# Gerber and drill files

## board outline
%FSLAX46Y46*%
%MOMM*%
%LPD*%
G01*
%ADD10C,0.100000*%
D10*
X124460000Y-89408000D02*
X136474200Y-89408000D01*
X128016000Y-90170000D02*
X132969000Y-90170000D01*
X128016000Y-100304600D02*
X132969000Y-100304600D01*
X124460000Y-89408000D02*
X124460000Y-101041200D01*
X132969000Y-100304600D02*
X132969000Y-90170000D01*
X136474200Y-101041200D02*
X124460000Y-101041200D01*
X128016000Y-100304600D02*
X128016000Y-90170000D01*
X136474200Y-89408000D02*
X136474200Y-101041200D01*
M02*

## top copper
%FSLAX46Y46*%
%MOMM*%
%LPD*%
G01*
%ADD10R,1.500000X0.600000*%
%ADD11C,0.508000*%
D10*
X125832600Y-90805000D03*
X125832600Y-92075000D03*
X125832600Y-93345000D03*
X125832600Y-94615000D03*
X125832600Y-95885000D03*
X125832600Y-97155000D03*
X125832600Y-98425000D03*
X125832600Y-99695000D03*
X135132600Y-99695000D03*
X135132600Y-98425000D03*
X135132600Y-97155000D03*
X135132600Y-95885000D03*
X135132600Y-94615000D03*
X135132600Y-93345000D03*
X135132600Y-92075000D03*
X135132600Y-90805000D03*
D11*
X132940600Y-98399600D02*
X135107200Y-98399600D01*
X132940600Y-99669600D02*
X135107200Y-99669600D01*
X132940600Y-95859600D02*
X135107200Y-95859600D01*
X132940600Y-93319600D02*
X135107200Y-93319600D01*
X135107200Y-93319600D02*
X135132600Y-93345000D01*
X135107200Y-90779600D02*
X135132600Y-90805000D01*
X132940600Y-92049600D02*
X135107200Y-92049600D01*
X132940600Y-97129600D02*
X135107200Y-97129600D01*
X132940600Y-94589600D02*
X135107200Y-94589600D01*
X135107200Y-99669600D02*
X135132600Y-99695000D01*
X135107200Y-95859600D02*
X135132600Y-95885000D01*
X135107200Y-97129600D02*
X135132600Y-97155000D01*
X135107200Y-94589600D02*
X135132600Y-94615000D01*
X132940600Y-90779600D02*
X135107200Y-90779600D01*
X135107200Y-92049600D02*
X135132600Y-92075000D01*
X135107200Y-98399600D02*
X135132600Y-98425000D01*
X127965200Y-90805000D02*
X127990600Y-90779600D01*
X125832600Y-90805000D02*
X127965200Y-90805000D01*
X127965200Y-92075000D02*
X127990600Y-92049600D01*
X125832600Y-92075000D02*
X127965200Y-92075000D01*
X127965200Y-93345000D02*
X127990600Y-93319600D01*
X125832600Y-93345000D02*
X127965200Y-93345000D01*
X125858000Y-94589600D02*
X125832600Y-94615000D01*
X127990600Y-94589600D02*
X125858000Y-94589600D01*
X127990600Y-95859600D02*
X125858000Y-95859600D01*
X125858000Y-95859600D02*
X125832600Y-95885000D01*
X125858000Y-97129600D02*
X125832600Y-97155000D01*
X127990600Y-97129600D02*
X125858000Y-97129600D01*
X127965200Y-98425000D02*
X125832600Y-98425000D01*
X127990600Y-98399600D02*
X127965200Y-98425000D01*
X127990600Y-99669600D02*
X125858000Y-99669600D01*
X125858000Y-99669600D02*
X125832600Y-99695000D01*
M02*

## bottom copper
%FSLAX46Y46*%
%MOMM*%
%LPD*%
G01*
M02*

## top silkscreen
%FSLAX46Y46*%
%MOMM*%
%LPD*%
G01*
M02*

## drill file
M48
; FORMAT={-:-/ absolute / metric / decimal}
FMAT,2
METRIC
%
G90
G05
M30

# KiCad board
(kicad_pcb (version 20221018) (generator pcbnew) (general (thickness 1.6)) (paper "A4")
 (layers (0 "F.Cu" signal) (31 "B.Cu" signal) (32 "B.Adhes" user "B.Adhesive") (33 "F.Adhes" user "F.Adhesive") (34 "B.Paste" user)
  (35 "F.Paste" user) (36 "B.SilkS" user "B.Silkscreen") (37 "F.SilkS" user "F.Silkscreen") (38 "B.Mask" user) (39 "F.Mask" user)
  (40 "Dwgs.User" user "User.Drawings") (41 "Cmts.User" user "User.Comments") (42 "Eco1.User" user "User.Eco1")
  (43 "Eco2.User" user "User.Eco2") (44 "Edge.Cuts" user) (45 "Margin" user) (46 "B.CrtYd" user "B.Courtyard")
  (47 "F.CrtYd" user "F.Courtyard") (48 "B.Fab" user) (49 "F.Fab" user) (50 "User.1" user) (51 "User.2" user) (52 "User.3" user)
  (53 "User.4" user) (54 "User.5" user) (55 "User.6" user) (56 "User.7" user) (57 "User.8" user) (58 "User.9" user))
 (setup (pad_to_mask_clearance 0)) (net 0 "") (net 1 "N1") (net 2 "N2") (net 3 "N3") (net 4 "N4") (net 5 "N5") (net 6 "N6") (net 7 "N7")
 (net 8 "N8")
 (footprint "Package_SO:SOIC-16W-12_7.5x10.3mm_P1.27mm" (layer "F.Cu") (at 130.4826 95.25)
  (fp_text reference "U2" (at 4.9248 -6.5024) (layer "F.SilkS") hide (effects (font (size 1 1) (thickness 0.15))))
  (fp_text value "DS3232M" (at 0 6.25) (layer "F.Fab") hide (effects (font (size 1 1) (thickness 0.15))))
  (pad "1" smd rect (at -4.65 -4.445) (size 1.5 0.6) (layers "F.Cu" "F.Paste" "F.Mask") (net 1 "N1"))
  (pad "2" smd rect (at -4.65 -3.175) (size 1.5 0.6) (layers "F.Cu" "F.Paste" "F.Mask") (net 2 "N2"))
  (pad "3" smd rect (at -4.65 -1.905) (size 1.5 0.6) (layers "F.Cu" "F.Paste" "F.Mask") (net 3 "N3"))
  (pad "4" smd rect (at -4.65 -0.635) (size 1.5 0.6) (layers "F.Cu" "F.Paste" "F.Mask"))
  (pad "5" smd rect (at -4.65 0.635) (size 1.5 0.6) (layers "F.Cu" "F.Paste" "F.Mask"))
  (pad "6" smd rect (at -4.65 1.905) (size 1.5 0.6) (layers "F.Cu" "F.Paste" "F.Mask") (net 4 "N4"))
  (pad "7" smd rect (at -4.65 3.175) (size 1.5 0.6) (layers "F.Cu" "F.Paste" "F.Mask") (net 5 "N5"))
  (pad "8" smd rect (at -4.65 4.445) (size 1.5 0.6) (layers "F.Cu" "F.Paste" "F.Mask") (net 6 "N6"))
  (pad "9" smd rect (at 4.65 4.445) (size 1.5 0.6) (layers "F.Cu" "F.Paste" "F.Mask"))
  (pad "10" smd rect (at 4.65 3.175) (size 1.5 0.6) (layers "F.Cu" "F.Paste" "F.Mask"))
  (pad "11" smd rect (at 4.65 1.905) (size 1.5 0.6) (layers "F.Cu" "F.Paste" "F.Mask"))
  (pad "12" smd rect (at 4.65 0.635) (size 1.5 0.6) (layers "F.Cu" "F.Paste" "F.Mask"))
  (pad "13" smd rect (at 4.65 -0.635) (size 1.5 0.6) (layers "F.Cu" "F.Paste" "F.Mask"))
  (pad "14" smd rect (at 4.65 -1.905) (size 1.5 0.6) (layers "F.Cu" "F.Paste" "F.Mask"))
  (pad "15" smd rect (at 4.65 -3.175) (size 1.5 0.6) (layers "F.Cu" "F.Paste" "F.Mask"))
  (pad "16" smd rect (at 4.65 -4.445) (size 1.5 0.6) (layers "F.Cu" "F.Paste" "F.Mask")))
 (gr_line (start 124.46 89.408) (end 136.4742 89.408) (stroke (width 0.1) (type default)) (layer "Edge.Cuts"))
 (gr_line (start 128.016 90.17) (end 132.969 90.17) (stroke (width 0.1) (type default)) (layer "Edge.Cuts"))
 (gr_line (start 128.016 100.3046) (end 132.969 100.3046) (stroke (width 0.1) (type default)) (layer "Edge.Cuts"))
 (gr_line (start 124.46 89.408) (end 124.46 101.0412) (stroke (width 0.1) (type default)) (layer "Edge.Cuts"))
 (gr_line (start 132.969 100.3046) (end 132.969 90.17) (stroke (width 0.1) (type default)) (layer "Edge.Cuts"))
 (gr_line (start 136.4742 101.0412) (end 124.46 101.0412) (stroke (width 0.1) (type default)) (layer "Edge.Cuts"))
 (gr_line (start 128.016 100.3046) (end 128.016 90.17) (stroke (width 0.1) (type default)) (layer "Edge.Cuts"))
 (gr_line (start 136.4742 89.408) (end 136.4742 101.0412) (stroke (width 0.1) (type default)) (layer "Edge.Cuts"))
 (segment (start 132.9406 98.3996) (end 135.1072 98.3996) (width 0.508) (layer "F.Cu") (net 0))
 (segment (start 132.9406 99.6696) (end 135.1072 99.6696) (width 0.508) (layer "F.Cu") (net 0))
 (segment (start 132.9406 95.8596) (end 135.1072 95.8596) (width 0.508) (layer "F.Cu") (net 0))
 (segment (start 132.9406 93.3196) (end 135.1072 93.3196) (width 0.508) (layer "F.Cu") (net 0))
 (segment (start 135.1072 93.3196) (end 135.1326 93.345) (width 0.508) (layer "F.Cu") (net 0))
 (segment (start 135.1072 90.7796) (end 135.1326 90.805) (width 0.508) (layer "F.Cu") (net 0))
 (segment (start 132.9406 92.0496) (end 135.1072 92.0496) (width 0.508) (layer "F.Cu") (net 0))
 (segment (start 132.9406 97.1296) (end 135.1072 97.1296) (width 0.508) (layer "F.Cu") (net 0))
 (segment (start 132.9406 94.5896) (end 135.1072 94.5896) (width 0.508) (layer "F.Cu") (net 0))
 (segment (start 135.1072 99.6696) (end 135.1326 99.695) (width 0.508) (layer "F.Cu") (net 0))
 (segment (start 135.1072 95.8596) (end 135.1326 95.885) (width 0.508) (layer "F.Cu") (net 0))
 (segment (start 135.1072 97.1296) (end 135.1326 97.155) (width 0.508) (layer "F.Cu") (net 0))
 (segment (start 135.1072 94.5896) (end 135.1326 94.615) (width 0.508) (layer "F.Cu") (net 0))
 (segment (start 132.9406 90.7796) (end 135.1072 90.7796) (width 0.508) (layer "F.Cu") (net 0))
 (segment (start 135.1072 92.0496) (end 135.1326 92.075) (width 0.508) (layer "F.Cu") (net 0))
 (segment (start 135.1072 98.3996) (end 135.1326 98.425) (width 0.508) (layer "F.Cu") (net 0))
 (segment (start 127.9652 90.805) (end 127.9906 90.7796) (width 0.508) (layer "F.Cu") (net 1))
 (segment (start 125.8326 90.805) (end 127.9652 90.805) (width 0.508) (layer "F.Cu") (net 1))
 (segment (start 127.9652 92.075) (end 127.9906 92.0496) (width 0.508) (layer "F.Cu") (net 2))
 (segment (start 125.8326 92.075) (end 127.9652 92.075) (width 0.508) (layer "F.Cu") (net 2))
 (segment (start 127.9652 93.345) (end 127.9906 93.3196) (width 0.508) (layer "F.Cu") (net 3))
 (segment (start 125.8326 93.345) (end 127.9652 93.345) (width 0.508) (layer "F.Cu") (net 3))
 (segment (start 125.858 94.5896) (end 125.8326 94.615) (width 0.508) (layer "F.Cu") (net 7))
 (segment (start 127.9906 94.5896) (end 125.858 94.5896) (width 0.508) (layer "F.Cu") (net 7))
 (segment (start 127.9906 95.8596) (end 125.858 95.8596) (width 0.508) (layer "F.Cu") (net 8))
 (segment (start 125.858 95.8596) (end 125.8326 95.885) (width 0.508) (layer "F.Cu") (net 8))
 (segment (start 125.858 97.1296) (end 125.8326 97.155) (width 0.508) (layer "F.Cu") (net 4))
 (segment (start 127.9906 97.1296) (end 125.858 97.1296) (width 0.508) (layer "F.Cu") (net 4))
 (segment (start 127.9652 98.425) (end 125.8326 98.425) (width 0.508) (layer "F.Cu") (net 5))
 (segment (start 127.9906 98.3996) (end 127.9652 98.425) (width 0.508) (layer "F.Cu") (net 5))
 (segment (start 127.9906 99.6696) (end 125.858 99.6696) (width 0.508) (layer "F.Cu") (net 6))
 (segment (start 125.858 99.6696) (end 125.8326 99.695) (width 0.508) (layer "F.Cu") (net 6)))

